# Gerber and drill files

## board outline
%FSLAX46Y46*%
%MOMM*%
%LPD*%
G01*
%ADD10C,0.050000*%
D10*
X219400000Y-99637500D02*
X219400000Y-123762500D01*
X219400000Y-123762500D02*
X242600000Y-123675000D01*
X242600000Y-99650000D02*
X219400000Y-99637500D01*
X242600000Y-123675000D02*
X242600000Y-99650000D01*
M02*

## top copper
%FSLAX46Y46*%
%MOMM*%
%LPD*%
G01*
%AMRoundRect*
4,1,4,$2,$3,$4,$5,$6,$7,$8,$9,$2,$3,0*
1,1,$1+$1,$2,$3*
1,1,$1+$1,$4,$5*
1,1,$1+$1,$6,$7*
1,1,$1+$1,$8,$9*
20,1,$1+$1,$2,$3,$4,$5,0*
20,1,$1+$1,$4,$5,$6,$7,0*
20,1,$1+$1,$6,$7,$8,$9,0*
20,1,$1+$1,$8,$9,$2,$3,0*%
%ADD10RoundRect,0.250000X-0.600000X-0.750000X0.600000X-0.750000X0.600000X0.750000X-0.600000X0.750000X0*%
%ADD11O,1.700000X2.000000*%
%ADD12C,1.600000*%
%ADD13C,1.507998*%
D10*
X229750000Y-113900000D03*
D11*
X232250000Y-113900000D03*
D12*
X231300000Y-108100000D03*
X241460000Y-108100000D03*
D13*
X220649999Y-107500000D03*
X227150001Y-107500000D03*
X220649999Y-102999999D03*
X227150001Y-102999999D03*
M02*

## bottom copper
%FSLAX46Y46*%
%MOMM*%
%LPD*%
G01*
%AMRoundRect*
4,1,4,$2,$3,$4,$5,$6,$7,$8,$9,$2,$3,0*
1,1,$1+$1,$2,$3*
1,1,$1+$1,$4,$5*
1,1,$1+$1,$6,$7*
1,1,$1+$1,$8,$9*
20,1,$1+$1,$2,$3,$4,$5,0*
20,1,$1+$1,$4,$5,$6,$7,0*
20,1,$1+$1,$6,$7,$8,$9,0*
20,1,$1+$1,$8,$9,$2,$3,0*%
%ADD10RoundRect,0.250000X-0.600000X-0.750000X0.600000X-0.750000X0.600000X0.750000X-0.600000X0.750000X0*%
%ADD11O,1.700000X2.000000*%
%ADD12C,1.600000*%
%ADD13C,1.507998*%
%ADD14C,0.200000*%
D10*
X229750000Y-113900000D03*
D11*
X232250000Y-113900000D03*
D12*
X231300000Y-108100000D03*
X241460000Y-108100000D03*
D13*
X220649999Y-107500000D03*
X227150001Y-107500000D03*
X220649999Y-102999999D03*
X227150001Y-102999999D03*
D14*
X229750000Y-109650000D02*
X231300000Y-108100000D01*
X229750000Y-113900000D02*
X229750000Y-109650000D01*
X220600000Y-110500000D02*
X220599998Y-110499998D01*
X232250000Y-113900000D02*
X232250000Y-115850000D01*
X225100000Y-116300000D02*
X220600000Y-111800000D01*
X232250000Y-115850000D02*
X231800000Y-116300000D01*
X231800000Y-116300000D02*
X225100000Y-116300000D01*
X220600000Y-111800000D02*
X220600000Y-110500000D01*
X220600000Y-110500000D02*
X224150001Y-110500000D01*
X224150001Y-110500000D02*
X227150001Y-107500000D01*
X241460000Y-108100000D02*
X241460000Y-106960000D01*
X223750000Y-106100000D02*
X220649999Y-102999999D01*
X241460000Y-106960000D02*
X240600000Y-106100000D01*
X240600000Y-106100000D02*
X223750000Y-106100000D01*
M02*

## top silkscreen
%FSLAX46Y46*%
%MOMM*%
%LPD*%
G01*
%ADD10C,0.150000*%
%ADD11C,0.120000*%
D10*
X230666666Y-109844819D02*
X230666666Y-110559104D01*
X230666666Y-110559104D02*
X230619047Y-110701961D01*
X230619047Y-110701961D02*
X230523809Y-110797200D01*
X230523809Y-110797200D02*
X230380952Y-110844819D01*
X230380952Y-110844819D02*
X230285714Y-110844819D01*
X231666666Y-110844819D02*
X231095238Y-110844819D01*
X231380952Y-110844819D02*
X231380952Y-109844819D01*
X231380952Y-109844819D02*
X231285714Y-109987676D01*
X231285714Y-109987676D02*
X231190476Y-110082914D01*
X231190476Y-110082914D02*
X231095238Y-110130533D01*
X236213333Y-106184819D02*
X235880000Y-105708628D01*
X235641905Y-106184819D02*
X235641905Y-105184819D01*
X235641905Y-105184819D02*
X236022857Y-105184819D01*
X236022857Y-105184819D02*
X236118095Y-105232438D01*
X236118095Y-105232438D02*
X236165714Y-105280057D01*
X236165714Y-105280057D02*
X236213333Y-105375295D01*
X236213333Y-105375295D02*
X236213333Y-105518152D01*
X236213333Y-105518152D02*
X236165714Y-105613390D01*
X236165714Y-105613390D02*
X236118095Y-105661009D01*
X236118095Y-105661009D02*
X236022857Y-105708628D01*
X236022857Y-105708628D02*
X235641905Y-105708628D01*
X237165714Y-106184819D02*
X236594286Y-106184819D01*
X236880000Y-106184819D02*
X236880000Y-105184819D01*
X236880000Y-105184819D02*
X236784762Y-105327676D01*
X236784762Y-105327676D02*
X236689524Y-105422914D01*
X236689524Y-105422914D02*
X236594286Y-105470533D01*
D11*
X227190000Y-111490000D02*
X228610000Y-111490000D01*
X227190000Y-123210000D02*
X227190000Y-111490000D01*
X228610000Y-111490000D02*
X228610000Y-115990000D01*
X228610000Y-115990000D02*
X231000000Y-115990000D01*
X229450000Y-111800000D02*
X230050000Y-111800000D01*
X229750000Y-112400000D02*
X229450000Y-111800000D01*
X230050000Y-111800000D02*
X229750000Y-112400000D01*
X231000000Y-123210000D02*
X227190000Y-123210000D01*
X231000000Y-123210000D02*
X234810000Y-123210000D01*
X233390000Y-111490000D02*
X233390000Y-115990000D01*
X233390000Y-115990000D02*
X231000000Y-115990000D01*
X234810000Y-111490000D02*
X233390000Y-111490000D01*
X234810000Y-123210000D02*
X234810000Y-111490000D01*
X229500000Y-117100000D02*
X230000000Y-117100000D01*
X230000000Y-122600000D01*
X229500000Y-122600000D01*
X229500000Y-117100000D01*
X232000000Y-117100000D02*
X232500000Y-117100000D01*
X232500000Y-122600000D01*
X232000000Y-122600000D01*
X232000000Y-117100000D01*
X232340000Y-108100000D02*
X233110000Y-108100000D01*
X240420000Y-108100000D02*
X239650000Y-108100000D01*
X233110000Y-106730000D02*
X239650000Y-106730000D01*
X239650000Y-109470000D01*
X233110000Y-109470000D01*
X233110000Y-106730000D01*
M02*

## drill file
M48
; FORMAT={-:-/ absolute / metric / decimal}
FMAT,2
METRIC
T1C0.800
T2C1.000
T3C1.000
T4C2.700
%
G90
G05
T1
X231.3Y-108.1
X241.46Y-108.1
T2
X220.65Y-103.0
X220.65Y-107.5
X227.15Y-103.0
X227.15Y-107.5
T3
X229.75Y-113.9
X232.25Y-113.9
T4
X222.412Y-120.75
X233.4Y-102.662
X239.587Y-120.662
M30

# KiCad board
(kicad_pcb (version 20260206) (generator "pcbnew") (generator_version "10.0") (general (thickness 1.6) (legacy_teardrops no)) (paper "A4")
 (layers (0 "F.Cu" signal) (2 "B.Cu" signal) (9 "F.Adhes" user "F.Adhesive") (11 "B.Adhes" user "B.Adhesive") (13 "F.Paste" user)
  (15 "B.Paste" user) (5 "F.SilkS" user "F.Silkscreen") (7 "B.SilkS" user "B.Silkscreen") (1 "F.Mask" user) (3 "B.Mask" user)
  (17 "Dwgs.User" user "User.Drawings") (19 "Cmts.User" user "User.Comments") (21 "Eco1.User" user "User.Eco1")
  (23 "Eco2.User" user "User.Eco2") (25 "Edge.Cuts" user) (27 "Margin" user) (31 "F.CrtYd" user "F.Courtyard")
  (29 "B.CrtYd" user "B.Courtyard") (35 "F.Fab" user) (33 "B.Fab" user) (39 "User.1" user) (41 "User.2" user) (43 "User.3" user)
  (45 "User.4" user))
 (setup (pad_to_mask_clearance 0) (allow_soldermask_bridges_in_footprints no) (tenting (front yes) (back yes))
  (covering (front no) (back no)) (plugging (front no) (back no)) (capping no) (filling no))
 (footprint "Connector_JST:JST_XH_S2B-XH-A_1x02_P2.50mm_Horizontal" (layer "F.Cu") (at 229.75 113.9)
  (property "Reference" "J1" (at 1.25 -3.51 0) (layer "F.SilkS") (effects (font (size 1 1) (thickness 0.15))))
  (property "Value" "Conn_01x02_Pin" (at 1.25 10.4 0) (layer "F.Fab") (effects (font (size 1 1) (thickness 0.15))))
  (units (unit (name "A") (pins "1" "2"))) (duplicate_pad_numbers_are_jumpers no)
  (fp_line (start -2.56 -2.41) (end -1.14 -2.41) (stroke (width 0.12) (type solid)) (layer "F.SilkS"))
  (fp_line (start -2.56 9.31) (end -2.56 -2.41) (stroke (width 0.12) (type solid)) (layer "F.SilkS"))
  (fp_line (start -1.14 -2.41) (end -1.14 2.09) (stroke (width 0.12) (type solid)) (layer "F.SilkS"))
  (fp_line (start -1.14 2.09) (end 1.25 2.09) (stroke (width 0.12) (type solid)) (layer "F.SilkS"))
  (fp_line (start -0.3 -2.1) (end 0.3 -2.1) (stroke (width 0.12) (type solid)) (layer "F.SilkS"))
  (fp_line (start 0 -1.5) (end -0.3 -2.1) (stroke (width 0.12) (type solid)) (layer "F.SilkS"))
  (fp_line (start 0.3 -2.1) (end 0 -1.5) (stroke (width 0.12) (type solid)) (layer "F.SilkS"))
  (fp_line (start 1.25 9.31) (end -2.56 9.31) (stroke (width 0.12) (type solid)) (layer "F.SilkS"))
  (fp_line (start 1.25 9.31) (end 5.06 9.31) (stroke (width 0.12) (type solid)) (layer "F.SilkS"))
  (fp_line (start 3.64 -2.41) (end 3.64 2.09) (stroke (width 0.12) (type solid)) (layer "F.SilkS"))
  (fp_line (start 3.64 2.09) (end 1.25 2.09) (stroke (width 0.12) (type solid)) (layer "F.SilkS"))
  (fp_line (start 5.06 -2.41) (end 3.64 -2.41) (stroke (width 0.12) (type solid)) (layer "F.SilkS"))
  (fp_line (start 5.06 9.31) (end 5.06 -2.41) (stroke (width 0.12) (type solid)) (layer "F.SilkS"))
  (fp_rect (start -0.25 3.2) (end 0.25 8.7) (stroke (width 0.12) (type solid)) (fill no) (layer "F.SilkS"))
  (fp_rect (start 2.25 3.2) (end 2.75 8.7) (stroke (width 0.12) (type solid)) (fill no) (layer "F.SilkS"))
  (pad "1" thru_hole roundrect (at 0 0) (size 1.7 2) (drill 1) (layers "*.Cu" "*.Mask") (remove_unused_layers no)
   (roundrect_rratio 0.147059) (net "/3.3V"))
  (pad "2" thru_hole oval (at 2.5 0) (size 1.7 2) (drill 1) (layers "*.Cu" "*.Mask") (remove_unused_layers no) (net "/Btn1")))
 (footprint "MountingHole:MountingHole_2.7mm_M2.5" (layer "F.Cu") (at 222.4125 120.75)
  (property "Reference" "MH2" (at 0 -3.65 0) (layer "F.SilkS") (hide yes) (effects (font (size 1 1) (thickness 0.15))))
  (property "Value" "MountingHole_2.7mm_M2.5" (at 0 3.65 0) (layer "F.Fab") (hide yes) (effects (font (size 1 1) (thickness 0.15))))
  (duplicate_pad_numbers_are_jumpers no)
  (pad "" np_thru_hole circle (at 0 0) (size 2.7 2.7) (drill 2.7) (layers "*.Cu" "*.Mask")))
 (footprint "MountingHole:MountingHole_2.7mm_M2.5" (layer "F.Cu") (at 239.5875 120.6625)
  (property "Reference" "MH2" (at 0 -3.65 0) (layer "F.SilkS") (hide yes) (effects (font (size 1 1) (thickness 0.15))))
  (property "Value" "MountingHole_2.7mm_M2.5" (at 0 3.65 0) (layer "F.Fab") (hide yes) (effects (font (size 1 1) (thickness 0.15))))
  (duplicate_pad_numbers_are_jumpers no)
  (pad "" np_thru_hole circle (at 0 0) (size 2.7 2.7) (drill 2.7) (layers "*.Cu" "*.Mask")))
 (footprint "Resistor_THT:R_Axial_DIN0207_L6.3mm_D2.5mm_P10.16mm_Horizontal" (layer "F.Cu") (at 231.3 108.1)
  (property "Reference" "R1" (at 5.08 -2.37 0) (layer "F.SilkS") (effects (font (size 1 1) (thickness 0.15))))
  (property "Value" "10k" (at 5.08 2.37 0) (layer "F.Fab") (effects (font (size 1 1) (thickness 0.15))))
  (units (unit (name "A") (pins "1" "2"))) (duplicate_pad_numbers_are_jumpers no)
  (fp_line (start 1.04 0) (end 1.81 0) (stroke (width 0.12) (type solid)) (layer "F.SilkS"))
  (fp_line (start 9.12 0) (end 8.35 0) (stroke (width 0.12) (type solid)) (layer "F.SilkS"))
  (fp_rect (start 1.81 -1.37) (end 8.35 1.37) (stroke (width 0.12) (type solid)) (fill no) (layer "F.SilkS"))
  (pad "1" thru_hole circle (at 0 0) (size 1.6 1.6) (drill 0.8) (layers "*.Cu" "*.Mask") (remove_unused_layers no) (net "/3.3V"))
  (pad "2" thru_hole circle (at 10.16 0) (size 1.6 1.6) (drill 0.8) (layers "*.Cu" "*.Mask") (remove_unused_layers no) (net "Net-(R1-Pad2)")))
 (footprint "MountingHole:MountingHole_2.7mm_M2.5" (layer "F.Cu") (at 233.4 102.6625)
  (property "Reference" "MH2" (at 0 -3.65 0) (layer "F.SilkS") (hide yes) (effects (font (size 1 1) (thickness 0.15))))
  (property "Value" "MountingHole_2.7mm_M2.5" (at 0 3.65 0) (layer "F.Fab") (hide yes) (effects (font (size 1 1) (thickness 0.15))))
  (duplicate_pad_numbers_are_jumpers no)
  (pad "" np_thru_hole circle (at 0 0) (size 2.7 2.7) (drill 2.7) (layers "*.Cu" "*.Mask")))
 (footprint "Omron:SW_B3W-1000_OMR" (layer "B.Cu") (at 220.649999 107.5)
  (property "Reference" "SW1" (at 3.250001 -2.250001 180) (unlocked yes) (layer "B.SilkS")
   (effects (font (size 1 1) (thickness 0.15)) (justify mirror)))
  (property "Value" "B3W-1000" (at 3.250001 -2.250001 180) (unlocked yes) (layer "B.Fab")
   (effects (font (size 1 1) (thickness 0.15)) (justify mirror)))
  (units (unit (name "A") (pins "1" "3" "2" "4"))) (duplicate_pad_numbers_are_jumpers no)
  (pad "1" thru_hole circle (at 0 0) (size 1.507998 1.507998) (drill 0.999998) (layers "*.Cu" "*.Mask") (remove_unused_layers no)
   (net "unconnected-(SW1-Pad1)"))
  (pad "2" thru_hole circle (at 6.500002 0) (size 1.507998 1.507998) (drill 0.999998) (layers "*.Cu" "*.Mask") (remove_unused_layers no)
   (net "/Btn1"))
  (pad "3" thru_hole circle (at 0 -4.500001) (size 1.507998 1.507998) (drill 0.999998) (layers "*.Cu" "*.Mask") (remove_unused_layers no)
   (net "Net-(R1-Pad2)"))
  (pad "4" thru_hole circle (at 6.500002 -4.500001) (size 1.507998 1.507998) (drill 0.999998) (layers "*.Cu" "*.Mask")
   (remove_unused_layers no) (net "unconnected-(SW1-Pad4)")))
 (gr_line (start 219.4 99.6375) (end 219.4 123.7625) (stroke (width 0.05) (type default)) (layer "Edge.Cuts"))
 (gr_line (start 219.4 123.7625) (end 242.6 123.675) (stroke (width 0.05) (type default)) (layer "Edge.Cuts"))
 (gr_line (start 242.6 99.65) (end 219.4 99.6375) (stroke (width 0.05) (type default)) (layer "Edge.Cuts"))
 (gr_line (start 242.6 123.675) (end 242.6 99.65) (stroke (width 0.05) (type default)) (layer "Edge.Cuts"))
 (segment (start 229.75 109.65) (end 231.3 108.1) (width 0.2) (layer "B.Cu") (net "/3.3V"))
 (segment (start 229.75 113.9) (end 229.75 109.65) (width 0.2) (layer "B.Cu") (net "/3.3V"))
 (segment (start 220.6 110.5) (end 220.599998 110.499998) (width 0.2) (layer "B.Cu") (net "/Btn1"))
 (segment (start 232.25 113.9) (end 232.25 115.85) (width 0.2) (layer "B.Cu") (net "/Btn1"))
 (segment (start 225.1 116.3) (end 220.6 111.8) (width 0.2) (layer "B.Cu") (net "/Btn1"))
 (segment (start 232.25 115.85) (end 231.8 116.3) (width 0.2) (layer "B.Cu") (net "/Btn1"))
 (segment (start 231.8 116.3) (end 225.1 116.3) (width 0.2) (layer "B.Cu") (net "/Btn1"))
 (segment (start 220.6 111.8) (end 220.6 110.5) (width 0.2) (layer "B.Cu") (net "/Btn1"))
 (segment (start 220.6 110.5) (end 224.150001 110.5) (width 0.2) (layer "B.Cu") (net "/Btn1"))
 (segment (start 224.150001 110.5) (end 227.150001 107.5) (width 0.2) (layer "B.Cu") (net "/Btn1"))
 (segment (start 241.46 108.1) (end 241.46 106.96) (width 0.2) (layer "B.Cu") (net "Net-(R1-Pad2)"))
 (segment (start 223.75 106.1) (end 220.649999 102.999999) (width 0.2) (layer "B.Cu") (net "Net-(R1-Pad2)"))
 (segment (start 241.46 106.96) (end 240.6 106.1) (width 0.2) (layer "B.Cu") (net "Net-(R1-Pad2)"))
 (segment (start 240.6 106.1) (end 223.75 106.1) (width 0.2) (layer "B.Cu") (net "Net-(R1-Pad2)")))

